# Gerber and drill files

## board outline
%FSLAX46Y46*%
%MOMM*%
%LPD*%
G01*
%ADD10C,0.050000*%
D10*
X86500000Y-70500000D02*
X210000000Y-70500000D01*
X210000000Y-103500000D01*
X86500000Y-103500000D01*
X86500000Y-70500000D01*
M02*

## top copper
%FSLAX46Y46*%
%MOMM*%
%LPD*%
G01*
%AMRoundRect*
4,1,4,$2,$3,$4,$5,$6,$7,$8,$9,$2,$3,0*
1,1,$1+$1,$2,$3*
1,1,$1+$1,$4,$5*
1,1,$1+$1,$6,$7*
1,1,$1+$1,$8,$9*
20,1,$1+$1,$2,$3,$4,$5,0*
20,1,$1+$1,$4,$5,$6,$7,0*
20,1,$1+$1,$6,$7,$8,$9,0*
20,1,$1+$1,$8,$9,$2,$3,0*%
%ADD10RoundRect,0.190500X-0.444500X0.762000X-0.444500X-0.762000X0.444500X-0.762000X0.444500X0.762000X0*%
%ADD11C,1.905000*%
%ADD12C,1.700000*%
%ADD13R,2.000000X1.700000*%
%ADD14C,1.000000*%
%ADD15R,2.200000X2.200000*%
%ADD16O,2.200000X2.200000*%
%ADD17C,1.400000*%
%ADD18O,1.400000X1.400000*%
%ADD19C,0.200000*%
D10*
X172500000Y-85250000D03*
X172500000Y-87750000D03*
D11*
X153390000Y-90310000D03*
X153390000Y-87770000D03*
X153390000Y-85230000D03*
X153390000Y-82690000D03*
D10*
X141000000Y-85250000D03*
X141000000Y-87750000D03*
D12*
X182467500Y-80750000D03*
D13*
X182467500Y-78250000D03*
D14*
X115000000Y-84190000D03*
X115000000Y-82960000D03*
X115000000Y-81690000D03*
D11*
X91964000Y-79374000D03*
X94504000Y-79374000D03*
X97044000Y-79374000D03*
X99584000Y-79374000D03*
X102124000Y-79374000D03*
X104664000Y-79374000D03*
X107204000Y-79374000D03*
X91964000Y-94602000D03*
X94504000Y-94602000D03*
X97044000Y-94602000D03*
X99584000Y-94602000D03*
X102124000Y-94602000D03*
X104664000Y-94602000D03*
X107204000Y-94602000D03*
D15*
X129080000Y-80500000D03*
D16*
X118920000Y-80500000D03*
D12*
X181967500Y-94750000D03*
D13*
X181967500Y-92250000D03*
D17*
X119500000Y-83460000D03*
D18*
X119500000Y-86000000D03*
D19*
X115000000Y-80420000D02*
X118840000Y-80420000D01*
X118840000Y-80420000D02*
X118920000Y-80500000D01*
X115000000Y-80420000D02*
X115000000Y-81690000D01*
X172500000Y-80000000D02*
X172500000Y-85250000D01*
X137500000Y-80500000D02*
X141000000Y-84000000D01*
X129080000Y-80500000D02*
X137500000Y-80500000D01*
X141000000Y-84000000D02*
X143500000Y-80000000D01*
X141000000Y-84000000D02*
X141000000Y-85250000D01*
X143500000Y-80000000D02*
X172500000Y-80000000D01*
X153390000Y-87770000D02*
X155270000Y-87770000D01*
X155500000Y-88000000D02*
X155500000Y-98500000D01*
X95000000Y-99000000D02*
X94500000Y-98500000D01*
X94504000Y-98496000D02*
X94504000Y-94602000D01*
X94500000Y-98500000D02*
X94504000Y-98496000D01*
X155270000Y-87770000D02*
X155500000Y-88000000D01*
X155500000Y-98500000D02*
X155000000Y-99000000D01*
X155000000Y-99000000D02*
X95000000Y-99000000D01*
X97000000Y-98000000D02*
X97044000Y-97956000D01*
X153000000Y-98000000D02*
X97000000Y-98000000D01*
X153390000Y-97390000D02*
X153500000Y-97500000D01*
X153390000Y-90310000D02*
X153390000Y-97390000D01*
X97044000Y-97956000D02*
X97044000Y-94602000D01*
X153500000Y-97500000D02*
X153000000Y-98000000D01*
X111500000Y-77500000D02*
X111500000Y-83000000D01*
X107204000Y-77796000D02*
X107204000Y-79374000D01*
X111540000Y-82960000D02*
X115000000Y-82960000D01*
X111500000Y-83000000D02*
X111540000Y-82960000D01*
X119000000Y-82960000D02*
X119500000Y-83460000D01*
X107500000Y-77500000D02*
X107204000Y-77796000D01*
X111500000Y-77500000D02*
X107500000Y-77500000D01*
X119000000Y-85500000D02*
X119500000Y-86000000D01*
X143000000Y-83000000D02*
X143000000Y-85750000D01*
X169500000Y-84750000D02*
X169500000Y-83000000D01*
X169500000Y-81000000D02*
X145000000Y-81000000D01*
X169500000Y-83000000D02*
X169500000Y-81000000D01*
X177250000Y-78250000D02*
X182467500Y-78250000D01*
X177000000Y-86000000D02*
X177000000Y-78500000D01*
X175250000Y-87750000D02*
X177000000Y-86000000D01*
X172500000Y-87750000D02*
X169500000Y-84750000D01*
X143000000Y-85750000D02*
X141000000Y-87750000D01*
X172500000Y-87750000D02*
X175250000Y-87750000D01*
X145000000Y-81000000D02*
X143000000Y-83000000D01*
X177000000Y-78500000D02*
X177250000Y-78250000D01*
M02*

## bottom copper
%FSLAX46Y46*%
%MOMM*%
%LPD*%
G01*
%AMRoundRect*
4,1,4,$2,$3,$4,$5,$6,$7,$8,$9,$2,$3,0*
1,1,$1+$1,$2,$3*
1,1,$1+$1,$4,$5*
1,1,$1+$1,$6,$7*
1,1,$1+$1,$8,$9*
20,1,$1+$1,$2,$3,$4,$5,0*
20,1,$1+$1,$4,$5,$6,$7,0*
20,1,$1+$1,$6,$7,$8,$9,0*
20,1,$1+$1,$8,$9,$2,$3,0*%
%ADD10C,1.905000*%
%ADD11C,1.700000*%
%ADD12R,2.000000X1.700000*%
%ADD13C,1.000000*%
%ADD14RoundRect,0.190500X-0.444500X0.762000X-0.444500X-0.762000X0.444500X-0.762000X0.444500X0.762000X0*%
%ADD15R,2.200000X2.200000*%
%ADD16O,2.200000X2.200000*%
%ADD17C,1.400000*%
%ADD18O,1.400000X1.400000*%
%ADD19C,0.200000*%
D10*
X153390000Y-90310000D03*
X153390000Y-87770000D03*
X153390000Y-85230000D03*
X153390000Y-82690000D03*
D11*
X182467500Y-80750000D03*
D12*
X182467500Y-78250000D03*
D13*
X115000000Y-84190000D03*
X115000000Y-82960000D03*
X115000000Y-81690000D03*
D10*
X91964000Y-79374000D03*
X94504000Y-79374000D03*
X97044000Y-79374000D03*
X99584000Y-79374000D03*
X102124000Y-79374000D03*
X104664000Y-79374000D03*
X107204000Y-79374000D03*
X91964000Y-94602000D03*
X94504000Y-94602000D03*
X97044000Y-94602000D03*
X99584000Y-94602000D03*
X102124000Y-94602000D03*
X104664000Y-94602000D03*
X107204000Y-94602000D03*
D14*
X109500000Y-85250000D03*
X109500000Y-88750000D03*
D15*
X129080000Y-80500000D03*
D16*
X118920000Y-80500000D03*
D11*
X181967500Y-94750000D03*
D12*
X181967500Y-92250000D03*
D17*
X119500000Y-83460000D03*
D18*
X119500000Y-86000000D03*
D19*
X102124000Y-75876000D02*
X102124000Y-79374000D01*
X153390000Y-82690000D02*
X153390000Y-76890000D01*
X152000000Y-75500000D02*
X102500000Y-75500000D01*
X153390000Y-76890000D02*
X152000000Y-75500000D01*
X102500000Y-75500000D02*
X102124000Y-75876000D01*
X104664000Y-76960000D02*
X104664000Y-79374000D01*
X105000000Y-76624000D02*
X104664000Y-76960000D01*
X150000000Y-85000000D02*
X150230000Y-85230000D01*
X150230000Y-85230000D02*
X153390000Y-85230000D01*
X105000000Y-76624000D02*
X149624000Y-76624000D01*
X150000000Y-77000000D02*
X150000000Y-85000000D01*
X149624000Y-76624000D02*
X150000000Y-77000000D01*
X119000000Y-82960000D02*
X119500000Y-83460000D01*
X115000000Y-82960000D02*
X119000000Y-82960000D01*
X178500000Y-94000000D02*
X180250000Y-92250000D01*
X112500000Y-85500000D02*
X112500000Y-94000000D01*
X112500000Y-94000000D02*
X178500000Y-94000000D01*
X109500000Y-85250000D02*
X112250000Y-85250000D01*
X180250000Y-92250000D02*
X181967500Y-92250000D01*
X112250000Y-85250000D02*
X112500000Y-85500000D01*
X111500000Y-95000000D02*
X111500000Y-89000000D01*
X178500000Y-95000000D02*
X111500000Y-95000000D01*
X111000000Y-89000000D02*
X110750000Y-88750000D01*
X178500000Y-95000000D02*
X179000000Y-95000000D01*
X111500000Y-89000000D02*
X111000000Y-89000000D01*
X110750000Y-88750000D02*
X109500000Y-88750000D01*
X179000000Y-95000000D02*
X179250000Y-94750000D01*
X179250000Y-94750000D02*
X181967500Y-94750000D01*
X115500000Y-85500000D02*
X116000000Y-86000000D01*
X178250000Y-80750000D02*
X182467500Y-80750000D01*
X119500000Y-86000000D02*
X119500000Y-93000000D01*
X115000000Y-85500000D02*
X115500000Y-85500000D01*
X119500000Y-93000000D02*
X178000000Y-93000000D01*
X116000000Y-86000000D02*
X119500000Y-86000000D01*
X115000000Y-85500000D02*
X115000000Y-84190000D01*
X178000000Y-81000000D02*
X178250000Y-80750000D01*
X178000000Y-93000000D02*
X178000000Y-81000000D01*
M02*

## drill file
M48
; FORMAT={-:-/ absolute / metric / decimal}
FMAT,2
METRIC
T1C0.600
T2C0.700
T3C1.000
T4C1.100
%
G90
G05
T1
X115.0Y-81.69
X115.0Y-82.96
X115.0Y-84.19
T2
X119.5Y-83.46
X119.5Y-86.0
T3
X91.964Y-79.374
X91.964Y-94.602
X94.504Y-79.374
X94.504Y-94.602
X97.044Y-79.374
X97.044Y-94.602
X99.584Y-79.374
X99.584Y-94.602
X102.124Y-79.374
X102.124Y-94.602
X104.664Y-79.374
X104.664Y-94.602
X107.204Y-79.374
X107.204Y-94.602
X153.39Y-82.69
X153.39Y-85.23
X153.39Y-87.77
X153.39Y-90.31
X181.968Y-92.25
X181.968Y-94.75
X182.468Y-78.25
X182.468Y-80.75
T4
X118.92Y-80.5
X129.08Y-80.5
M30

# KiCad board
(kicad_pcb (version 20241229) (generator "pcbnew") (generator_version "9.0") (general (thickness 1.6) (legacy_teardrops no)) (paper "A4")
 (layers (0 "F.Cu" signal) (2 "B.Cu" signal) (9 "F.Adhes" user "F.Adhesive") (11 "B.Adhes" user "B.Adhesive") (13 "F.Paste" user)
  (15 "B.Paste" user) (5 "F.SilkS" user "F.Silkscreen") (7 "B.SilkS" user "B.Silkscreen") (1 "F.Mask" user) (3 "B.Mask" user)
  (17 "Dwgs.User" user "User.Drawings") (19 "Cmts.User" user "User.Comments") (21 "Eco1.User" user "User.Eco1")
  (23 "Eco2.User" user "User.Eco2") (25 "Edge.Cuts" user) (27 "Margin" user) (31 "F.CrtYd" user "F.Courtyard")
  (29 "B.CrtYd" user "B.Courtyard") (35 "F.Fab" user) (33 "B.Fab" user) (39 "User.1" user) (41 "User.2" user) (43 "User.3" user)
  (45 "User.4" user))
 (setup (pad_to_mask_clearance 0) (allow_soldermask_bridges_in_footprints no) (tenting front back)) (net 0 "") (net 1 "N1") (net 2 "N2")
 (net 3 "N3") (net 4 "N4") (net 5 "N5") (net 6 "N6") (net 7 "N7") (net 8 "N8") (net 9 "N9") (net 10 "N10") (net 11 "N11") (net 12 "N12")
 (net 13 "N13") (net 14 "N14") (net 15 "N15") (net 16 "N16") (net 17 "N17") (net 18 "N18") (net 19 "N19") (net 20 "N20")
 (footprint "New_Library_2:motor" (layer "F.Cu") (at 172.5 86.5 -90)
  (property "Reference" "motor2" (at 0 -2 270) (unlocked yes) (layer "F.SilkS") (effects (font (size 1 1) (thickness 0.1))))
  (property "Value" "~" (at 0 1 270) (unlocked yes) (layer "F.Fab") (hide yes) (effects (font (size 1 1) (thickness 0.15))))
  (pad "1" connect roundrect (at -1.25 0 270) (size 1.905 1.27) (layers "F.Cu" "F.Mask") (roundrect_rratio 0.15) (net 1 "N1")
   (thermal_bridge_angle 45))
  (pad "2" connect roundrect (at 1.25 0 270) (size 1.905 1.27) (layers "F.Cu" "F.Mask") (roundrect_rratio 0.15) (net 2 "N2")
   (thermal_bridge_angle 45)))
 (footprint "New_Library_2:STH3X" (layer "F.Cu") (at 152.1 86.5 90)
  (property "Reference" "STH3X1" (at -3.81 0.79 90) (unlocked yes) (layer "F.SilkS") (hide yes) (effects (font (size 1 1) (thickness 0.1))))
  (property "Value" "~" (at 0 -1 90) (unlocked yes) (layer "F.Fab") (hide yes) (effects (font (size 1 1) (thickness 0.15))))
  (pad "1" thru_hole circle (at -3.81 1.29 180) (size 1.905 1.905) (drill 1) (layers "*.Cu" "*.Mask") (remove_unused_layers no) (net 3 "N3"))
  (pad "2" thru_hole circle (at -1.27 1.29 90) (size 1.905 1.905) (drill 1) (layers "*.Cu" "*.Mask") (remove_unused_layers no) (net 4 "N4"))
  (pad "3" thru_hole circle (at 1.27 1.29 90) (size 1.905 1.905) (drill 1) (layers "*.Cu" "*.Mask") (remove_unused_layers no) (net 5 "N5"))
  (pad "4" thru_hole circle (at 3.81 1.29 90) (size 1.905 1.905) (drill 1) (layers "*.Cu" "*.Mask") (remove_unused_layers no) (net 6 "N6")))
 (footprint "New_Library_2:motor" (layer "F.Cu") (at 141 86.5 -90)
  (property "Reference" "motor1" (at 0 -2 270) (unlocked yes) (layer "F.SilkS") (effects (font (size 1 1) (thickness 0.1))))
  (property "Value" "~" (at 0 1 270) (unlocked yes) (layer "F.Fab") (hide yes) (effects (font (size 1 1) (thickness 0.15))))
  (pad "1" connect roundrect (at -1.25 0 270) (size 1.905 1.27) (layers "F.Cu" "F.Mask") (roundrect_rratio 0.15) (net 1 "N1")
   (thermal_bridge_angle 45))
  (pad "2" connect roundrect (at 1.25 0 270) (size 1.905 1.27) (layers "F.Cu" "F.Mask") (roundrect_rratio 0.15) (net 2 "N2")
   (thermal_bridge_angle 45)))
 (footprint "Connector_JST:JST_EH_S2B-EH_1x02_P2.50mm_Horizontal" (layer "B.Cu") (at 182.4675 80.75 90)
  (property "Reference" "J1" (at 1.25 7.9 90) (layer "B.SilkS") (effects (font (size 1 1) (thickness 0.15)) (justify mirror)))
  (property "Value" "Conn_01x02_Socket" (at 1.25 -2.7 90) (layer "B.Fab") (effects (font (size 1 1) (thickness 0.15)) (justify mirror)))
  (pad "1" thru_hole circle (at 0 0 90) (size 1.7 1.7) (drill 1) (layers "*.Cu" "*.Mask") (remove_unused_layers no) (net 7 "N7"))
  (pad "2" thru_hole rect (at 2.5 0 90) (size 1.7 2) (drill 1) (layers "*.Cu" "*.Mask") (remove_unused_layers no) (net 2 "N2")))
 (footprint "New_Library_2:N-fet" (layer "B.Cu") (at 115 82.96 90)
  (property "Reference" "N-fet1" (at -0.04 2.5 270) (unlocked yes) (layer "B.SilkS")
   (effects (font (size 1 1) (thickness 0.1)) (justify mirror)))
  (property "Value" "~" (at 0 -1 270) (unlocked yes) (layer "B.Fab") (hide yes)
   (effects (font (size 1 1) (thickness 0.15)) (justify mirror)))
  (pad "1" thru_hole circle (at -1.23 0 90) (size 1 1) (drill 0.6) (layers "*.Cu" "*.Mask") (remove_unused_layers no) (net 7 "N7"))
  (pad "2" thru_hole circle (at 0 0 90) (size 1 1) (drill 0.6) (layers "*.Cu" "*.Mask") (remove_unused_layers no) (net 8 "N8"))
  (pad "3" thru_hole circle (at 1.27 0 90) (size 1 1) (drill 0.6) (layers "*.Cu" "*.Mask") (remove_unused_layers no) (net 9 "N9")))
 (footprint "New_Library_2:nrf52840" (layer "B.Cu") (at 92 87 -90)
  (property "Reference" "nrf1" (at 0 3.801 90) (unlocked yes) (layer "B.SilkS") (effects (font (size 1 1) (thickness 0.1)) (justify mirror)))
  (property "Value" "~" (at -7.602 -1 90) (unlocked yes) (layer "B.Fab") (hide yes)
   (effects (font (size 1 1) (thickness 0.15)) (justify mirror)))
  (pad "1" thru_hole circle (at -7.626 0.036 270) (size 1.905 1.905) (drill 1) (layers "*.Cu" "*.Mask") (remove_unused_layers no)
   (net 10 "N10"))
  (pad "2" thru_hole circle (at -7.626 -2.504 270) (size 1.905 1.905) (drill 1) (layers "*.Cu" "*.Mask") (remove_unused_layers no)
   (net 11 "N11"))
  (pad "3" thru_hole circle (at -7.626 -5.044 270) (size 1.905 1.905) (drill 1) (layers "*.Cu" "*.Mask") (remove_unused_layers no)
   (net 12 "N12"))
  (pad "4" thru_hole circle (at -7.626 -7.584 270) (size 1.905 1.905) (drill 1) (layers "*.Cu" "*.Mask") (remove_unused_layers no)
   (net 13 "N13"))
  (pad "5" thru_hole circle (at -7.626 -10.124 270) (size 1.905 1.905) (drill 1) (layers "*.Cu" "*.Mask") (remove_unused_layers no)
   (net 6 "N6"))
  (pad "6" thru_hole circle (at -7.626 -12.664 270) (size 1.905 1.905) (drill 1) (layers "*.Cu" "*.Mask") (remove_unused_layers no)
   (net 5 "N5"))
  (pad "7" thru_hole circle (at -7.626 -15.204 270) (size 1.905 1.905) (drill 1) (layers "*.Cu" "*.Mask") (remove_unused_layers no)
   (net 8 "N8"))
  (pad "8" thru_hole circle (at 7.602 0.036 270) (size 1.905 1.905) (drill 1) (layers "*.Cu" "*.Mask") (remove_unused_layers no)
   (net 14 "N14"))
  (pad "9" thru_hole circle (at 7.602 -2.504 270) (size 1.905 1.905) (drill 1) (layers "*.Cu" "*.Mask") (remove_unused_layers no)
   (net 4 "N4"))
  (pad "10" thru_hole circle (at 7.602 -5.044 270) (size 1.905 1.905) (drill 1) (layers "*.Cu" "*.Mask") (remove_unused_layers no)
   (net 3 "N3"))
  (pad "11" thru_hole circle (at 7.602 -7.584 270) (size 1.905 1.905) (drill 1) (layers "*.Cu" "*.Mask") (remove_unused_layers no)
   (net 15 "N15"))
  (pad "12" thru_hole circle (at 7.602 -10.124 270) (size 1.905 1.905) (drill 1) (layers "*.Cu" "*.Mask") (remove_unused_layers no)
   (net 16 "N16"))
  (pad "13" thru_hole circle (at 7.602 -12.664 270) (size 1.905 1.905) (drill 1) (layers "*.Cu" "*.Mask") (remove_unused_layers no)
   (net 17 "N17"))
  (pad "14" thru_hole circle (at 7.602 -15.204 270) (size 1.905 1.905) (drill 1) (layers "*.Cu" "*.Mask") (remove_unused_layers no)
   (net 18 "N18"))
  (pad "15" smd roundrect (at -1.75 -17.5 270) (size 1.905 1.27) (layers "B.Cu" "B.Mask" "B.Paste") (roundrect_rratio 0.15) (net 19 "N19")
   (thermal_bridge_angle 45))
  (pad "16" smd roundrect (at 1.75 -17.5 270) (size 1.905 1.27) (layers "B.Cu" "B.Mask" "B.Paste") (roundrect_rratio 0.15) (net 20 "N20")
   (thermal_bridge_angle 45)))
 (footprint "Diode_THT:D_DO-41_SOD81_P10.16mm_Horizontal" (layer "B.Cu") (at 129.08 80.5 180)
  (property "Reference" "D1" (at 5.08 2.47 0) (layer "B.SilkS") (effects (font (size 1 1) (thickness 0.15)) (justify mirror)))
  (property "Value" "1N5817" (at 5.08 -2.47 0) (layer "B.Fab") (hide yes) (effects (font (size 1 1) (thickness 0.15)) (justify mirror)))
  (pad "1" thru_hole rect (at 0 0 180) (size 2.2 2.2) (drill 1.1) (layers "*.Cu" "*.Mask") (remove_unused_layers no) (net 1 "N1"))
  (pad "2" thru_hole oval (at 10.16 0 180) (size 2.2 2.2) (drill 1.1) (layers "*.Cu" "*.Mask") (remove_unused_layers no) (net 9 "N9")))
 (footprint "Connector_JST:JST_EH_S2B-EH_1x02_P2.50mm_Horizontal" (layer "B.Cu") (at 181.9675 94.75 90)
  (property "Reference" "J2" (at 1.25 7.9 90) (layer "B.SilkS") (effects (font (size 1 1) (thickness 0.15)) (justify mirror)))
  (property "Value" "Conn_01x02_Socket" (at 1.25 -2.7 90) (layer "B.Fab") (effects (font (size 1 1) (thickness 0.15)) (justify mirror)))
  (pad "1" thru_hole circle (at 0 0 90) (size 1.7 1.7) (drill 1) (layers "*.Cu" "*.Mask") (remove_unused_layers no) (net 20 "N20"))
  (pad "2" thru_hole rect (at 2.5 0 90) (size 1.7 2) (drill 1) (layers "*.Cu" "*.Mask") (remove_unused_layers no) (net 19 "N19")))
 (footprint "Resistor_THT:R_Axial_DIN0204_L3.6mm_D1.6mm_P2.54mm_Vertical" (layer "B.Cu") (at 119.5 83.46 -90)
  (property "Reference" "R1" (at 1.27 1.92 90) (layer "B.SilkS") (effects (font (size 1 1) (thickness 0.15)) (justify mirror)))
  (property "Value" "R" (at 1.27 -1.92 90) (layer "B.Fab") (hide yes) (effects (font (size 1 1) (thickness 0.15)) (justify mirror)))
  (pad "1" thru_hole circle (at 0 0 270) (size 1.4 1.4) (drill 0.7) (layers "*.Cu" "*.Mask") (remove_unused_layers no) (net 8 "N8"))
  (pad "2" thru_hole oval (at 2.54 0 270) (size 1.4 1.4) (drill 0.7) (layers "*.Cu" "*.Mask") (remove_unused_layers no) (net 7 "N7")))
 (gr_rect (start 86.5 70.5) (end 210 103.5) (stroke (width 0.05) (type default)) (fill no) (layer "Edge.Cuts"))
 (segment (start 115 80.42) (end 118.84 80.42) (width 0.2) (layer "F.Cu") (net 9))
 (segment (start 118.84 80.42) (end 118.92 80.5) (width 0.2) (layer "F.Cu") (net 9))
 (segment (start 115 80.42) (end 115 81.69) (width 0.2) (layer "F.Cu") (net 9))
 (segment (start 172.5 80) (end 172.5 85.25) (width 0.2) (layer "F.Cu") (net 1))
 (segment (start 137.5 80.5) (end 141 84) (width 0.2) (layer "F.Cu") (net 1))
 (segment (start 129.08 80.5) (end 137.5 80.5) (width 0.2) (layer "F.Cu") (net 1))
 (segment (start 141 84) (end 143.5 80) (width 0.2) (layer "F.Cu") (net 1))
 (segment (start 141 84) (end 141 85.25) (width 0.2) (layer "F.Cu") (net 1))
 (segment (start 143.5 80) (end 172.5 80) (width 0.2) (layer "F.Cu") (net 1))
 (segment (start 102.124 75.876) (end 102.124 79.374) (width 0.2) (layer "B.Cu") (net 6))
 (segment (start 153.39 82.69) (end 153.39 76.89) (width 0.2) (layer "B.Cu") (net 6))
 (segment (start 152 75.5) (end 102.5 75.5) (width 0.2) (layer "B.Cu") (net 6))
 (segment (start 153.39 76.89) (end 152 75.5) (width 0.2) (layer "B.Cu") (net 6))
 (segment (start 102.5 75.5) (end 102.124 75.876) (width 0.2) (layer "B.Cu") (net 6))
 (segment (start 153.39 87.77) (end 155.27 87.77) (width 0.2) (layer "F.Cu") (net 4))
 (segment (start 155.5 88) (end 155.5 98.5) (width 0.2) (layer "F.Cu") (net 4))
 (segment (start 95 99) (end 94.5 98.5) (width 0.2) (layer "F.Cu") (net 4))
 (segment (start 94.504 98.496) (end 94.504 94.602) (width 0.2) (layer "F.Cu") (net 4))
 (segment (start 94.5 98.5) (end 94.504 98.496) (width 0.2) (layer "F.Cu") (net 4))
 (segment (start 155.27 87.77) (end 155.5 88) (width 0.2) (layer "F.Cu") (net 4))
 (segment (start 155.5 98.5) (end 155 99) (width 0.2) (layer "F.Cu") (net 4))
 (segment (start 155 99) (end 95 99) (width 0.2) (layer "F.Cu") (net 4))
 (segment (start 97 98) (end 97.044 97.956) (width 0.2) (layer "F.Cu") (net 3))
 (segment (start 153 98) (end 97 98) (width 0.2) (layer "F.Cu") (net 3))
 (segment (start 153.39 97.39) (end 153.5 97.5) (width 0.2) (layer "F.Cu") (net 3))
 (segment (start 153.39 90.31) (end 153.39 97.39) (width 0.2) (layer "F.Cu") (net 3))
 (segment (start 97.044 97.956) (end 97.044 94.602) (width 0.2) (layer "F.Cu") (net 3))
 (segment (start 153.5 97.5) (end 153 98) (width 0.2) (layer "F.Cu") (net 3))
 (segment (start 104.664 76.96) (end 104.664 79.374) (width 0.2) (layer "B.Cu") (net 5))
 (segment (start 105 76.624) (end 104.664 76.96) (width 0.2) (layer "B.Cu") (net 5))
 (segment (start 150 85) (end 150.23 85.23) (width 0.2) (layer "B.Cu") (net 5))
 (segment (start 150.23 85.23) (end 153.39 85.23) (width 0.2) (layer "B.Cu") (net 5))
 (segment (start 105 76.624) (end 149.624 76.624) (width 0.2) (layer "B.Cu") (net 5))
 (segment (start 150 77) (end 150 85) (width 0.2) (layer "B.Cu") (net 5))
 (segment (start 149.624 76.624) (end 150 77) (width 0.2) (layer "B.Cu") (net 5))
 (segment (start 111.5 77.5) (end 111.5 83) (width 0.2) (layer "F.Cu") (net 8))
 (segment (start 107.204 77.796) (end 107.204 79.374) (width 0.2) (layer "F.Cu") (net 8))
 (segment (start 111.54 82.96) (end 115 82.96) (width 0.2) (layer "F.Cu") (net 8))
 (segment (start 111.5 83) (end 111.54 82.96) (width 0.2) (layer "F.Cu") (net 8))
 (segment (start 119 82.96) (end 119.5 83.46) (width 0.2) (layer "F.Cu") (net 8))
 (segment (start 107.5 77.5) (end 107.204 77.796) (width 0.2) (layer "F.Cu") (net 8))
 (segment (start 111.5 77.5) (end 107.5 77.5) (width 0.2) (layer "F.Cu") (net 8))
 (segment (start 119 82.96) (end 119.5 83.46) (width 0.2) (layer "B.Cu") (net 8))
 (segment (start 115 82.96) (end 119 82.96) (width 0.2) (layer "B.Cu") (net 8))
 (segment (start 178.5 94) (end 180.25 92.25) (width 0.2) (layer "B.Cu") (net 19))
 (segment (start 112.5 85.5) (end 112.5 94) (width 0.2) (layer "B.Cu") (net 19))
 (segment (start 112.5 94) (end 178.5 94) (width 0.2) (layer "B.Cu") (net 19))
 (segment (start 109.5 85.25) (end 112.25 85.25) (width 0.2) (layer "B.Cu") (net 19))
 (segment (start 180.25 92.25) (end 181.9675 92.25) (width 0.2) (layer "B.Cu") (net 19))
 (segment (start 112.25 85.25) (end 112.5 85.5) (width 0.2) (layer "B.Cu") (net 19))
 (segment (start 111.5 95) (end 111.5 89) (width 0.2) (layer "B.Cu") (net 20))
 (segment (start 178.5 95) (end 111.5 95) (width 0.2) (layer "B.Cu") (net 20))
 (segment (start 111 89) (end 110.75 88.75) (width 0.2) (layer "B.Cu") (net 20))
 (segment (start 178.5 95) (end 179 95) (width 0.2) (layer "B.Cu") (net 20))
 (segment (start 111.5 89) (end 111 89) (width 0.2) (layer "B.Cu") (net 20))
 (segment (start 110.75 88.75) (end 109.5 88.75) (width 0.2) (layer "B.Cu") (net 20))
 (segment (start 179 95) (end 179.25 94.75) (width 0.2) (layer "B.Cu") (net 20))
 (segment (start 179.25 94.75) (end 181.9675 94.75) (width 0.2) (layer "B.Cu") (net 20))
 (segment (start 119 85.5) (end 119.5 86) (width 0.2) (layer "F.Cu") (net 7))
 (segment (start 115.5 85.5) (end 116 86) (width 0.2) (layer "B.Cu") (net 7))
 (segment (start 178.25 80.75) (end 182.4675 80.75) (width 0.2) (layer "B.Cu") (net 7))
 (segment (start 119.5 86) (end 119.5 93) (width 0.2) (layer "B.Cu") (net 7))
 (segment (start 115 85.5) (end 115.5 85.5) (width 0.2) (layer "B.Cu") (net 7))
 (segment (start 119.5 93) (end 178 93) (width 0.2) (layer "B.Cu") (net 7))
 (segment (start 116 86) (end 119.5 86) (width 0.2) (layer "B.Cu") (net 7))
 (segment (start 115 85.5) (end 115 84.19) (width 0.2) (layer "B.Cu") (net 7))
 (segment (start 178 81) (end 178.25 80.75) (width 0.2) (layer "B.Cu") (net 7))
 (segment (start 178 93) (end 178 81) (width 0.2) (layer "B.Cu") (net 7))
 (segment (start 143 83) (end 143 85.75) (width 0.2) (layer "F.Cu") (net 2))
 (segment (start 169.5 84.75) (end 169.5 83) (width 0.2) (layer "F.Cu") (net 2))
 (segment (start 169.5 81) (end 145 81) (width 0.2) (layer "F.Cu") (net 2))
 (segment (start 169.5 83) (end 169.5 81) (width 0.2) (layer "F.Cu") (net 2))
 (segment (start 177.25 78.25) (end 182.4675 78.25) (width 0.2) (layer "F.Cu") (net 2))
 (segment (start 177 86) (end 177 78.5) (width 0.2) (layer "F.Cu") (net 2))
 (segment (start 175.25 87.75) (end 177 86) (width 0.2) (layer "F.Cu") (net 2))
 (segment (start 172.5 87.75) (end 169.5 84.75) (width 0.2) (layer "F.Cu") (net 2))
 (segment (start 143 85.75) (end 141 87.75) (width 0.2) (layer "F.Cu") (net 2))
 (segment (start 172.5 87.75) (end 175.25 87.75) (width 0.2) (layer "F.Cu") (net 2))
 (segment (start 145 81) (end 143 83) (width 0.2) (layer "F.Cu") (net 2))
 (segment (start 177 78.5) (end 177.25 78.25) (width 0.2) (layer "F.Cu") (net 2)))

